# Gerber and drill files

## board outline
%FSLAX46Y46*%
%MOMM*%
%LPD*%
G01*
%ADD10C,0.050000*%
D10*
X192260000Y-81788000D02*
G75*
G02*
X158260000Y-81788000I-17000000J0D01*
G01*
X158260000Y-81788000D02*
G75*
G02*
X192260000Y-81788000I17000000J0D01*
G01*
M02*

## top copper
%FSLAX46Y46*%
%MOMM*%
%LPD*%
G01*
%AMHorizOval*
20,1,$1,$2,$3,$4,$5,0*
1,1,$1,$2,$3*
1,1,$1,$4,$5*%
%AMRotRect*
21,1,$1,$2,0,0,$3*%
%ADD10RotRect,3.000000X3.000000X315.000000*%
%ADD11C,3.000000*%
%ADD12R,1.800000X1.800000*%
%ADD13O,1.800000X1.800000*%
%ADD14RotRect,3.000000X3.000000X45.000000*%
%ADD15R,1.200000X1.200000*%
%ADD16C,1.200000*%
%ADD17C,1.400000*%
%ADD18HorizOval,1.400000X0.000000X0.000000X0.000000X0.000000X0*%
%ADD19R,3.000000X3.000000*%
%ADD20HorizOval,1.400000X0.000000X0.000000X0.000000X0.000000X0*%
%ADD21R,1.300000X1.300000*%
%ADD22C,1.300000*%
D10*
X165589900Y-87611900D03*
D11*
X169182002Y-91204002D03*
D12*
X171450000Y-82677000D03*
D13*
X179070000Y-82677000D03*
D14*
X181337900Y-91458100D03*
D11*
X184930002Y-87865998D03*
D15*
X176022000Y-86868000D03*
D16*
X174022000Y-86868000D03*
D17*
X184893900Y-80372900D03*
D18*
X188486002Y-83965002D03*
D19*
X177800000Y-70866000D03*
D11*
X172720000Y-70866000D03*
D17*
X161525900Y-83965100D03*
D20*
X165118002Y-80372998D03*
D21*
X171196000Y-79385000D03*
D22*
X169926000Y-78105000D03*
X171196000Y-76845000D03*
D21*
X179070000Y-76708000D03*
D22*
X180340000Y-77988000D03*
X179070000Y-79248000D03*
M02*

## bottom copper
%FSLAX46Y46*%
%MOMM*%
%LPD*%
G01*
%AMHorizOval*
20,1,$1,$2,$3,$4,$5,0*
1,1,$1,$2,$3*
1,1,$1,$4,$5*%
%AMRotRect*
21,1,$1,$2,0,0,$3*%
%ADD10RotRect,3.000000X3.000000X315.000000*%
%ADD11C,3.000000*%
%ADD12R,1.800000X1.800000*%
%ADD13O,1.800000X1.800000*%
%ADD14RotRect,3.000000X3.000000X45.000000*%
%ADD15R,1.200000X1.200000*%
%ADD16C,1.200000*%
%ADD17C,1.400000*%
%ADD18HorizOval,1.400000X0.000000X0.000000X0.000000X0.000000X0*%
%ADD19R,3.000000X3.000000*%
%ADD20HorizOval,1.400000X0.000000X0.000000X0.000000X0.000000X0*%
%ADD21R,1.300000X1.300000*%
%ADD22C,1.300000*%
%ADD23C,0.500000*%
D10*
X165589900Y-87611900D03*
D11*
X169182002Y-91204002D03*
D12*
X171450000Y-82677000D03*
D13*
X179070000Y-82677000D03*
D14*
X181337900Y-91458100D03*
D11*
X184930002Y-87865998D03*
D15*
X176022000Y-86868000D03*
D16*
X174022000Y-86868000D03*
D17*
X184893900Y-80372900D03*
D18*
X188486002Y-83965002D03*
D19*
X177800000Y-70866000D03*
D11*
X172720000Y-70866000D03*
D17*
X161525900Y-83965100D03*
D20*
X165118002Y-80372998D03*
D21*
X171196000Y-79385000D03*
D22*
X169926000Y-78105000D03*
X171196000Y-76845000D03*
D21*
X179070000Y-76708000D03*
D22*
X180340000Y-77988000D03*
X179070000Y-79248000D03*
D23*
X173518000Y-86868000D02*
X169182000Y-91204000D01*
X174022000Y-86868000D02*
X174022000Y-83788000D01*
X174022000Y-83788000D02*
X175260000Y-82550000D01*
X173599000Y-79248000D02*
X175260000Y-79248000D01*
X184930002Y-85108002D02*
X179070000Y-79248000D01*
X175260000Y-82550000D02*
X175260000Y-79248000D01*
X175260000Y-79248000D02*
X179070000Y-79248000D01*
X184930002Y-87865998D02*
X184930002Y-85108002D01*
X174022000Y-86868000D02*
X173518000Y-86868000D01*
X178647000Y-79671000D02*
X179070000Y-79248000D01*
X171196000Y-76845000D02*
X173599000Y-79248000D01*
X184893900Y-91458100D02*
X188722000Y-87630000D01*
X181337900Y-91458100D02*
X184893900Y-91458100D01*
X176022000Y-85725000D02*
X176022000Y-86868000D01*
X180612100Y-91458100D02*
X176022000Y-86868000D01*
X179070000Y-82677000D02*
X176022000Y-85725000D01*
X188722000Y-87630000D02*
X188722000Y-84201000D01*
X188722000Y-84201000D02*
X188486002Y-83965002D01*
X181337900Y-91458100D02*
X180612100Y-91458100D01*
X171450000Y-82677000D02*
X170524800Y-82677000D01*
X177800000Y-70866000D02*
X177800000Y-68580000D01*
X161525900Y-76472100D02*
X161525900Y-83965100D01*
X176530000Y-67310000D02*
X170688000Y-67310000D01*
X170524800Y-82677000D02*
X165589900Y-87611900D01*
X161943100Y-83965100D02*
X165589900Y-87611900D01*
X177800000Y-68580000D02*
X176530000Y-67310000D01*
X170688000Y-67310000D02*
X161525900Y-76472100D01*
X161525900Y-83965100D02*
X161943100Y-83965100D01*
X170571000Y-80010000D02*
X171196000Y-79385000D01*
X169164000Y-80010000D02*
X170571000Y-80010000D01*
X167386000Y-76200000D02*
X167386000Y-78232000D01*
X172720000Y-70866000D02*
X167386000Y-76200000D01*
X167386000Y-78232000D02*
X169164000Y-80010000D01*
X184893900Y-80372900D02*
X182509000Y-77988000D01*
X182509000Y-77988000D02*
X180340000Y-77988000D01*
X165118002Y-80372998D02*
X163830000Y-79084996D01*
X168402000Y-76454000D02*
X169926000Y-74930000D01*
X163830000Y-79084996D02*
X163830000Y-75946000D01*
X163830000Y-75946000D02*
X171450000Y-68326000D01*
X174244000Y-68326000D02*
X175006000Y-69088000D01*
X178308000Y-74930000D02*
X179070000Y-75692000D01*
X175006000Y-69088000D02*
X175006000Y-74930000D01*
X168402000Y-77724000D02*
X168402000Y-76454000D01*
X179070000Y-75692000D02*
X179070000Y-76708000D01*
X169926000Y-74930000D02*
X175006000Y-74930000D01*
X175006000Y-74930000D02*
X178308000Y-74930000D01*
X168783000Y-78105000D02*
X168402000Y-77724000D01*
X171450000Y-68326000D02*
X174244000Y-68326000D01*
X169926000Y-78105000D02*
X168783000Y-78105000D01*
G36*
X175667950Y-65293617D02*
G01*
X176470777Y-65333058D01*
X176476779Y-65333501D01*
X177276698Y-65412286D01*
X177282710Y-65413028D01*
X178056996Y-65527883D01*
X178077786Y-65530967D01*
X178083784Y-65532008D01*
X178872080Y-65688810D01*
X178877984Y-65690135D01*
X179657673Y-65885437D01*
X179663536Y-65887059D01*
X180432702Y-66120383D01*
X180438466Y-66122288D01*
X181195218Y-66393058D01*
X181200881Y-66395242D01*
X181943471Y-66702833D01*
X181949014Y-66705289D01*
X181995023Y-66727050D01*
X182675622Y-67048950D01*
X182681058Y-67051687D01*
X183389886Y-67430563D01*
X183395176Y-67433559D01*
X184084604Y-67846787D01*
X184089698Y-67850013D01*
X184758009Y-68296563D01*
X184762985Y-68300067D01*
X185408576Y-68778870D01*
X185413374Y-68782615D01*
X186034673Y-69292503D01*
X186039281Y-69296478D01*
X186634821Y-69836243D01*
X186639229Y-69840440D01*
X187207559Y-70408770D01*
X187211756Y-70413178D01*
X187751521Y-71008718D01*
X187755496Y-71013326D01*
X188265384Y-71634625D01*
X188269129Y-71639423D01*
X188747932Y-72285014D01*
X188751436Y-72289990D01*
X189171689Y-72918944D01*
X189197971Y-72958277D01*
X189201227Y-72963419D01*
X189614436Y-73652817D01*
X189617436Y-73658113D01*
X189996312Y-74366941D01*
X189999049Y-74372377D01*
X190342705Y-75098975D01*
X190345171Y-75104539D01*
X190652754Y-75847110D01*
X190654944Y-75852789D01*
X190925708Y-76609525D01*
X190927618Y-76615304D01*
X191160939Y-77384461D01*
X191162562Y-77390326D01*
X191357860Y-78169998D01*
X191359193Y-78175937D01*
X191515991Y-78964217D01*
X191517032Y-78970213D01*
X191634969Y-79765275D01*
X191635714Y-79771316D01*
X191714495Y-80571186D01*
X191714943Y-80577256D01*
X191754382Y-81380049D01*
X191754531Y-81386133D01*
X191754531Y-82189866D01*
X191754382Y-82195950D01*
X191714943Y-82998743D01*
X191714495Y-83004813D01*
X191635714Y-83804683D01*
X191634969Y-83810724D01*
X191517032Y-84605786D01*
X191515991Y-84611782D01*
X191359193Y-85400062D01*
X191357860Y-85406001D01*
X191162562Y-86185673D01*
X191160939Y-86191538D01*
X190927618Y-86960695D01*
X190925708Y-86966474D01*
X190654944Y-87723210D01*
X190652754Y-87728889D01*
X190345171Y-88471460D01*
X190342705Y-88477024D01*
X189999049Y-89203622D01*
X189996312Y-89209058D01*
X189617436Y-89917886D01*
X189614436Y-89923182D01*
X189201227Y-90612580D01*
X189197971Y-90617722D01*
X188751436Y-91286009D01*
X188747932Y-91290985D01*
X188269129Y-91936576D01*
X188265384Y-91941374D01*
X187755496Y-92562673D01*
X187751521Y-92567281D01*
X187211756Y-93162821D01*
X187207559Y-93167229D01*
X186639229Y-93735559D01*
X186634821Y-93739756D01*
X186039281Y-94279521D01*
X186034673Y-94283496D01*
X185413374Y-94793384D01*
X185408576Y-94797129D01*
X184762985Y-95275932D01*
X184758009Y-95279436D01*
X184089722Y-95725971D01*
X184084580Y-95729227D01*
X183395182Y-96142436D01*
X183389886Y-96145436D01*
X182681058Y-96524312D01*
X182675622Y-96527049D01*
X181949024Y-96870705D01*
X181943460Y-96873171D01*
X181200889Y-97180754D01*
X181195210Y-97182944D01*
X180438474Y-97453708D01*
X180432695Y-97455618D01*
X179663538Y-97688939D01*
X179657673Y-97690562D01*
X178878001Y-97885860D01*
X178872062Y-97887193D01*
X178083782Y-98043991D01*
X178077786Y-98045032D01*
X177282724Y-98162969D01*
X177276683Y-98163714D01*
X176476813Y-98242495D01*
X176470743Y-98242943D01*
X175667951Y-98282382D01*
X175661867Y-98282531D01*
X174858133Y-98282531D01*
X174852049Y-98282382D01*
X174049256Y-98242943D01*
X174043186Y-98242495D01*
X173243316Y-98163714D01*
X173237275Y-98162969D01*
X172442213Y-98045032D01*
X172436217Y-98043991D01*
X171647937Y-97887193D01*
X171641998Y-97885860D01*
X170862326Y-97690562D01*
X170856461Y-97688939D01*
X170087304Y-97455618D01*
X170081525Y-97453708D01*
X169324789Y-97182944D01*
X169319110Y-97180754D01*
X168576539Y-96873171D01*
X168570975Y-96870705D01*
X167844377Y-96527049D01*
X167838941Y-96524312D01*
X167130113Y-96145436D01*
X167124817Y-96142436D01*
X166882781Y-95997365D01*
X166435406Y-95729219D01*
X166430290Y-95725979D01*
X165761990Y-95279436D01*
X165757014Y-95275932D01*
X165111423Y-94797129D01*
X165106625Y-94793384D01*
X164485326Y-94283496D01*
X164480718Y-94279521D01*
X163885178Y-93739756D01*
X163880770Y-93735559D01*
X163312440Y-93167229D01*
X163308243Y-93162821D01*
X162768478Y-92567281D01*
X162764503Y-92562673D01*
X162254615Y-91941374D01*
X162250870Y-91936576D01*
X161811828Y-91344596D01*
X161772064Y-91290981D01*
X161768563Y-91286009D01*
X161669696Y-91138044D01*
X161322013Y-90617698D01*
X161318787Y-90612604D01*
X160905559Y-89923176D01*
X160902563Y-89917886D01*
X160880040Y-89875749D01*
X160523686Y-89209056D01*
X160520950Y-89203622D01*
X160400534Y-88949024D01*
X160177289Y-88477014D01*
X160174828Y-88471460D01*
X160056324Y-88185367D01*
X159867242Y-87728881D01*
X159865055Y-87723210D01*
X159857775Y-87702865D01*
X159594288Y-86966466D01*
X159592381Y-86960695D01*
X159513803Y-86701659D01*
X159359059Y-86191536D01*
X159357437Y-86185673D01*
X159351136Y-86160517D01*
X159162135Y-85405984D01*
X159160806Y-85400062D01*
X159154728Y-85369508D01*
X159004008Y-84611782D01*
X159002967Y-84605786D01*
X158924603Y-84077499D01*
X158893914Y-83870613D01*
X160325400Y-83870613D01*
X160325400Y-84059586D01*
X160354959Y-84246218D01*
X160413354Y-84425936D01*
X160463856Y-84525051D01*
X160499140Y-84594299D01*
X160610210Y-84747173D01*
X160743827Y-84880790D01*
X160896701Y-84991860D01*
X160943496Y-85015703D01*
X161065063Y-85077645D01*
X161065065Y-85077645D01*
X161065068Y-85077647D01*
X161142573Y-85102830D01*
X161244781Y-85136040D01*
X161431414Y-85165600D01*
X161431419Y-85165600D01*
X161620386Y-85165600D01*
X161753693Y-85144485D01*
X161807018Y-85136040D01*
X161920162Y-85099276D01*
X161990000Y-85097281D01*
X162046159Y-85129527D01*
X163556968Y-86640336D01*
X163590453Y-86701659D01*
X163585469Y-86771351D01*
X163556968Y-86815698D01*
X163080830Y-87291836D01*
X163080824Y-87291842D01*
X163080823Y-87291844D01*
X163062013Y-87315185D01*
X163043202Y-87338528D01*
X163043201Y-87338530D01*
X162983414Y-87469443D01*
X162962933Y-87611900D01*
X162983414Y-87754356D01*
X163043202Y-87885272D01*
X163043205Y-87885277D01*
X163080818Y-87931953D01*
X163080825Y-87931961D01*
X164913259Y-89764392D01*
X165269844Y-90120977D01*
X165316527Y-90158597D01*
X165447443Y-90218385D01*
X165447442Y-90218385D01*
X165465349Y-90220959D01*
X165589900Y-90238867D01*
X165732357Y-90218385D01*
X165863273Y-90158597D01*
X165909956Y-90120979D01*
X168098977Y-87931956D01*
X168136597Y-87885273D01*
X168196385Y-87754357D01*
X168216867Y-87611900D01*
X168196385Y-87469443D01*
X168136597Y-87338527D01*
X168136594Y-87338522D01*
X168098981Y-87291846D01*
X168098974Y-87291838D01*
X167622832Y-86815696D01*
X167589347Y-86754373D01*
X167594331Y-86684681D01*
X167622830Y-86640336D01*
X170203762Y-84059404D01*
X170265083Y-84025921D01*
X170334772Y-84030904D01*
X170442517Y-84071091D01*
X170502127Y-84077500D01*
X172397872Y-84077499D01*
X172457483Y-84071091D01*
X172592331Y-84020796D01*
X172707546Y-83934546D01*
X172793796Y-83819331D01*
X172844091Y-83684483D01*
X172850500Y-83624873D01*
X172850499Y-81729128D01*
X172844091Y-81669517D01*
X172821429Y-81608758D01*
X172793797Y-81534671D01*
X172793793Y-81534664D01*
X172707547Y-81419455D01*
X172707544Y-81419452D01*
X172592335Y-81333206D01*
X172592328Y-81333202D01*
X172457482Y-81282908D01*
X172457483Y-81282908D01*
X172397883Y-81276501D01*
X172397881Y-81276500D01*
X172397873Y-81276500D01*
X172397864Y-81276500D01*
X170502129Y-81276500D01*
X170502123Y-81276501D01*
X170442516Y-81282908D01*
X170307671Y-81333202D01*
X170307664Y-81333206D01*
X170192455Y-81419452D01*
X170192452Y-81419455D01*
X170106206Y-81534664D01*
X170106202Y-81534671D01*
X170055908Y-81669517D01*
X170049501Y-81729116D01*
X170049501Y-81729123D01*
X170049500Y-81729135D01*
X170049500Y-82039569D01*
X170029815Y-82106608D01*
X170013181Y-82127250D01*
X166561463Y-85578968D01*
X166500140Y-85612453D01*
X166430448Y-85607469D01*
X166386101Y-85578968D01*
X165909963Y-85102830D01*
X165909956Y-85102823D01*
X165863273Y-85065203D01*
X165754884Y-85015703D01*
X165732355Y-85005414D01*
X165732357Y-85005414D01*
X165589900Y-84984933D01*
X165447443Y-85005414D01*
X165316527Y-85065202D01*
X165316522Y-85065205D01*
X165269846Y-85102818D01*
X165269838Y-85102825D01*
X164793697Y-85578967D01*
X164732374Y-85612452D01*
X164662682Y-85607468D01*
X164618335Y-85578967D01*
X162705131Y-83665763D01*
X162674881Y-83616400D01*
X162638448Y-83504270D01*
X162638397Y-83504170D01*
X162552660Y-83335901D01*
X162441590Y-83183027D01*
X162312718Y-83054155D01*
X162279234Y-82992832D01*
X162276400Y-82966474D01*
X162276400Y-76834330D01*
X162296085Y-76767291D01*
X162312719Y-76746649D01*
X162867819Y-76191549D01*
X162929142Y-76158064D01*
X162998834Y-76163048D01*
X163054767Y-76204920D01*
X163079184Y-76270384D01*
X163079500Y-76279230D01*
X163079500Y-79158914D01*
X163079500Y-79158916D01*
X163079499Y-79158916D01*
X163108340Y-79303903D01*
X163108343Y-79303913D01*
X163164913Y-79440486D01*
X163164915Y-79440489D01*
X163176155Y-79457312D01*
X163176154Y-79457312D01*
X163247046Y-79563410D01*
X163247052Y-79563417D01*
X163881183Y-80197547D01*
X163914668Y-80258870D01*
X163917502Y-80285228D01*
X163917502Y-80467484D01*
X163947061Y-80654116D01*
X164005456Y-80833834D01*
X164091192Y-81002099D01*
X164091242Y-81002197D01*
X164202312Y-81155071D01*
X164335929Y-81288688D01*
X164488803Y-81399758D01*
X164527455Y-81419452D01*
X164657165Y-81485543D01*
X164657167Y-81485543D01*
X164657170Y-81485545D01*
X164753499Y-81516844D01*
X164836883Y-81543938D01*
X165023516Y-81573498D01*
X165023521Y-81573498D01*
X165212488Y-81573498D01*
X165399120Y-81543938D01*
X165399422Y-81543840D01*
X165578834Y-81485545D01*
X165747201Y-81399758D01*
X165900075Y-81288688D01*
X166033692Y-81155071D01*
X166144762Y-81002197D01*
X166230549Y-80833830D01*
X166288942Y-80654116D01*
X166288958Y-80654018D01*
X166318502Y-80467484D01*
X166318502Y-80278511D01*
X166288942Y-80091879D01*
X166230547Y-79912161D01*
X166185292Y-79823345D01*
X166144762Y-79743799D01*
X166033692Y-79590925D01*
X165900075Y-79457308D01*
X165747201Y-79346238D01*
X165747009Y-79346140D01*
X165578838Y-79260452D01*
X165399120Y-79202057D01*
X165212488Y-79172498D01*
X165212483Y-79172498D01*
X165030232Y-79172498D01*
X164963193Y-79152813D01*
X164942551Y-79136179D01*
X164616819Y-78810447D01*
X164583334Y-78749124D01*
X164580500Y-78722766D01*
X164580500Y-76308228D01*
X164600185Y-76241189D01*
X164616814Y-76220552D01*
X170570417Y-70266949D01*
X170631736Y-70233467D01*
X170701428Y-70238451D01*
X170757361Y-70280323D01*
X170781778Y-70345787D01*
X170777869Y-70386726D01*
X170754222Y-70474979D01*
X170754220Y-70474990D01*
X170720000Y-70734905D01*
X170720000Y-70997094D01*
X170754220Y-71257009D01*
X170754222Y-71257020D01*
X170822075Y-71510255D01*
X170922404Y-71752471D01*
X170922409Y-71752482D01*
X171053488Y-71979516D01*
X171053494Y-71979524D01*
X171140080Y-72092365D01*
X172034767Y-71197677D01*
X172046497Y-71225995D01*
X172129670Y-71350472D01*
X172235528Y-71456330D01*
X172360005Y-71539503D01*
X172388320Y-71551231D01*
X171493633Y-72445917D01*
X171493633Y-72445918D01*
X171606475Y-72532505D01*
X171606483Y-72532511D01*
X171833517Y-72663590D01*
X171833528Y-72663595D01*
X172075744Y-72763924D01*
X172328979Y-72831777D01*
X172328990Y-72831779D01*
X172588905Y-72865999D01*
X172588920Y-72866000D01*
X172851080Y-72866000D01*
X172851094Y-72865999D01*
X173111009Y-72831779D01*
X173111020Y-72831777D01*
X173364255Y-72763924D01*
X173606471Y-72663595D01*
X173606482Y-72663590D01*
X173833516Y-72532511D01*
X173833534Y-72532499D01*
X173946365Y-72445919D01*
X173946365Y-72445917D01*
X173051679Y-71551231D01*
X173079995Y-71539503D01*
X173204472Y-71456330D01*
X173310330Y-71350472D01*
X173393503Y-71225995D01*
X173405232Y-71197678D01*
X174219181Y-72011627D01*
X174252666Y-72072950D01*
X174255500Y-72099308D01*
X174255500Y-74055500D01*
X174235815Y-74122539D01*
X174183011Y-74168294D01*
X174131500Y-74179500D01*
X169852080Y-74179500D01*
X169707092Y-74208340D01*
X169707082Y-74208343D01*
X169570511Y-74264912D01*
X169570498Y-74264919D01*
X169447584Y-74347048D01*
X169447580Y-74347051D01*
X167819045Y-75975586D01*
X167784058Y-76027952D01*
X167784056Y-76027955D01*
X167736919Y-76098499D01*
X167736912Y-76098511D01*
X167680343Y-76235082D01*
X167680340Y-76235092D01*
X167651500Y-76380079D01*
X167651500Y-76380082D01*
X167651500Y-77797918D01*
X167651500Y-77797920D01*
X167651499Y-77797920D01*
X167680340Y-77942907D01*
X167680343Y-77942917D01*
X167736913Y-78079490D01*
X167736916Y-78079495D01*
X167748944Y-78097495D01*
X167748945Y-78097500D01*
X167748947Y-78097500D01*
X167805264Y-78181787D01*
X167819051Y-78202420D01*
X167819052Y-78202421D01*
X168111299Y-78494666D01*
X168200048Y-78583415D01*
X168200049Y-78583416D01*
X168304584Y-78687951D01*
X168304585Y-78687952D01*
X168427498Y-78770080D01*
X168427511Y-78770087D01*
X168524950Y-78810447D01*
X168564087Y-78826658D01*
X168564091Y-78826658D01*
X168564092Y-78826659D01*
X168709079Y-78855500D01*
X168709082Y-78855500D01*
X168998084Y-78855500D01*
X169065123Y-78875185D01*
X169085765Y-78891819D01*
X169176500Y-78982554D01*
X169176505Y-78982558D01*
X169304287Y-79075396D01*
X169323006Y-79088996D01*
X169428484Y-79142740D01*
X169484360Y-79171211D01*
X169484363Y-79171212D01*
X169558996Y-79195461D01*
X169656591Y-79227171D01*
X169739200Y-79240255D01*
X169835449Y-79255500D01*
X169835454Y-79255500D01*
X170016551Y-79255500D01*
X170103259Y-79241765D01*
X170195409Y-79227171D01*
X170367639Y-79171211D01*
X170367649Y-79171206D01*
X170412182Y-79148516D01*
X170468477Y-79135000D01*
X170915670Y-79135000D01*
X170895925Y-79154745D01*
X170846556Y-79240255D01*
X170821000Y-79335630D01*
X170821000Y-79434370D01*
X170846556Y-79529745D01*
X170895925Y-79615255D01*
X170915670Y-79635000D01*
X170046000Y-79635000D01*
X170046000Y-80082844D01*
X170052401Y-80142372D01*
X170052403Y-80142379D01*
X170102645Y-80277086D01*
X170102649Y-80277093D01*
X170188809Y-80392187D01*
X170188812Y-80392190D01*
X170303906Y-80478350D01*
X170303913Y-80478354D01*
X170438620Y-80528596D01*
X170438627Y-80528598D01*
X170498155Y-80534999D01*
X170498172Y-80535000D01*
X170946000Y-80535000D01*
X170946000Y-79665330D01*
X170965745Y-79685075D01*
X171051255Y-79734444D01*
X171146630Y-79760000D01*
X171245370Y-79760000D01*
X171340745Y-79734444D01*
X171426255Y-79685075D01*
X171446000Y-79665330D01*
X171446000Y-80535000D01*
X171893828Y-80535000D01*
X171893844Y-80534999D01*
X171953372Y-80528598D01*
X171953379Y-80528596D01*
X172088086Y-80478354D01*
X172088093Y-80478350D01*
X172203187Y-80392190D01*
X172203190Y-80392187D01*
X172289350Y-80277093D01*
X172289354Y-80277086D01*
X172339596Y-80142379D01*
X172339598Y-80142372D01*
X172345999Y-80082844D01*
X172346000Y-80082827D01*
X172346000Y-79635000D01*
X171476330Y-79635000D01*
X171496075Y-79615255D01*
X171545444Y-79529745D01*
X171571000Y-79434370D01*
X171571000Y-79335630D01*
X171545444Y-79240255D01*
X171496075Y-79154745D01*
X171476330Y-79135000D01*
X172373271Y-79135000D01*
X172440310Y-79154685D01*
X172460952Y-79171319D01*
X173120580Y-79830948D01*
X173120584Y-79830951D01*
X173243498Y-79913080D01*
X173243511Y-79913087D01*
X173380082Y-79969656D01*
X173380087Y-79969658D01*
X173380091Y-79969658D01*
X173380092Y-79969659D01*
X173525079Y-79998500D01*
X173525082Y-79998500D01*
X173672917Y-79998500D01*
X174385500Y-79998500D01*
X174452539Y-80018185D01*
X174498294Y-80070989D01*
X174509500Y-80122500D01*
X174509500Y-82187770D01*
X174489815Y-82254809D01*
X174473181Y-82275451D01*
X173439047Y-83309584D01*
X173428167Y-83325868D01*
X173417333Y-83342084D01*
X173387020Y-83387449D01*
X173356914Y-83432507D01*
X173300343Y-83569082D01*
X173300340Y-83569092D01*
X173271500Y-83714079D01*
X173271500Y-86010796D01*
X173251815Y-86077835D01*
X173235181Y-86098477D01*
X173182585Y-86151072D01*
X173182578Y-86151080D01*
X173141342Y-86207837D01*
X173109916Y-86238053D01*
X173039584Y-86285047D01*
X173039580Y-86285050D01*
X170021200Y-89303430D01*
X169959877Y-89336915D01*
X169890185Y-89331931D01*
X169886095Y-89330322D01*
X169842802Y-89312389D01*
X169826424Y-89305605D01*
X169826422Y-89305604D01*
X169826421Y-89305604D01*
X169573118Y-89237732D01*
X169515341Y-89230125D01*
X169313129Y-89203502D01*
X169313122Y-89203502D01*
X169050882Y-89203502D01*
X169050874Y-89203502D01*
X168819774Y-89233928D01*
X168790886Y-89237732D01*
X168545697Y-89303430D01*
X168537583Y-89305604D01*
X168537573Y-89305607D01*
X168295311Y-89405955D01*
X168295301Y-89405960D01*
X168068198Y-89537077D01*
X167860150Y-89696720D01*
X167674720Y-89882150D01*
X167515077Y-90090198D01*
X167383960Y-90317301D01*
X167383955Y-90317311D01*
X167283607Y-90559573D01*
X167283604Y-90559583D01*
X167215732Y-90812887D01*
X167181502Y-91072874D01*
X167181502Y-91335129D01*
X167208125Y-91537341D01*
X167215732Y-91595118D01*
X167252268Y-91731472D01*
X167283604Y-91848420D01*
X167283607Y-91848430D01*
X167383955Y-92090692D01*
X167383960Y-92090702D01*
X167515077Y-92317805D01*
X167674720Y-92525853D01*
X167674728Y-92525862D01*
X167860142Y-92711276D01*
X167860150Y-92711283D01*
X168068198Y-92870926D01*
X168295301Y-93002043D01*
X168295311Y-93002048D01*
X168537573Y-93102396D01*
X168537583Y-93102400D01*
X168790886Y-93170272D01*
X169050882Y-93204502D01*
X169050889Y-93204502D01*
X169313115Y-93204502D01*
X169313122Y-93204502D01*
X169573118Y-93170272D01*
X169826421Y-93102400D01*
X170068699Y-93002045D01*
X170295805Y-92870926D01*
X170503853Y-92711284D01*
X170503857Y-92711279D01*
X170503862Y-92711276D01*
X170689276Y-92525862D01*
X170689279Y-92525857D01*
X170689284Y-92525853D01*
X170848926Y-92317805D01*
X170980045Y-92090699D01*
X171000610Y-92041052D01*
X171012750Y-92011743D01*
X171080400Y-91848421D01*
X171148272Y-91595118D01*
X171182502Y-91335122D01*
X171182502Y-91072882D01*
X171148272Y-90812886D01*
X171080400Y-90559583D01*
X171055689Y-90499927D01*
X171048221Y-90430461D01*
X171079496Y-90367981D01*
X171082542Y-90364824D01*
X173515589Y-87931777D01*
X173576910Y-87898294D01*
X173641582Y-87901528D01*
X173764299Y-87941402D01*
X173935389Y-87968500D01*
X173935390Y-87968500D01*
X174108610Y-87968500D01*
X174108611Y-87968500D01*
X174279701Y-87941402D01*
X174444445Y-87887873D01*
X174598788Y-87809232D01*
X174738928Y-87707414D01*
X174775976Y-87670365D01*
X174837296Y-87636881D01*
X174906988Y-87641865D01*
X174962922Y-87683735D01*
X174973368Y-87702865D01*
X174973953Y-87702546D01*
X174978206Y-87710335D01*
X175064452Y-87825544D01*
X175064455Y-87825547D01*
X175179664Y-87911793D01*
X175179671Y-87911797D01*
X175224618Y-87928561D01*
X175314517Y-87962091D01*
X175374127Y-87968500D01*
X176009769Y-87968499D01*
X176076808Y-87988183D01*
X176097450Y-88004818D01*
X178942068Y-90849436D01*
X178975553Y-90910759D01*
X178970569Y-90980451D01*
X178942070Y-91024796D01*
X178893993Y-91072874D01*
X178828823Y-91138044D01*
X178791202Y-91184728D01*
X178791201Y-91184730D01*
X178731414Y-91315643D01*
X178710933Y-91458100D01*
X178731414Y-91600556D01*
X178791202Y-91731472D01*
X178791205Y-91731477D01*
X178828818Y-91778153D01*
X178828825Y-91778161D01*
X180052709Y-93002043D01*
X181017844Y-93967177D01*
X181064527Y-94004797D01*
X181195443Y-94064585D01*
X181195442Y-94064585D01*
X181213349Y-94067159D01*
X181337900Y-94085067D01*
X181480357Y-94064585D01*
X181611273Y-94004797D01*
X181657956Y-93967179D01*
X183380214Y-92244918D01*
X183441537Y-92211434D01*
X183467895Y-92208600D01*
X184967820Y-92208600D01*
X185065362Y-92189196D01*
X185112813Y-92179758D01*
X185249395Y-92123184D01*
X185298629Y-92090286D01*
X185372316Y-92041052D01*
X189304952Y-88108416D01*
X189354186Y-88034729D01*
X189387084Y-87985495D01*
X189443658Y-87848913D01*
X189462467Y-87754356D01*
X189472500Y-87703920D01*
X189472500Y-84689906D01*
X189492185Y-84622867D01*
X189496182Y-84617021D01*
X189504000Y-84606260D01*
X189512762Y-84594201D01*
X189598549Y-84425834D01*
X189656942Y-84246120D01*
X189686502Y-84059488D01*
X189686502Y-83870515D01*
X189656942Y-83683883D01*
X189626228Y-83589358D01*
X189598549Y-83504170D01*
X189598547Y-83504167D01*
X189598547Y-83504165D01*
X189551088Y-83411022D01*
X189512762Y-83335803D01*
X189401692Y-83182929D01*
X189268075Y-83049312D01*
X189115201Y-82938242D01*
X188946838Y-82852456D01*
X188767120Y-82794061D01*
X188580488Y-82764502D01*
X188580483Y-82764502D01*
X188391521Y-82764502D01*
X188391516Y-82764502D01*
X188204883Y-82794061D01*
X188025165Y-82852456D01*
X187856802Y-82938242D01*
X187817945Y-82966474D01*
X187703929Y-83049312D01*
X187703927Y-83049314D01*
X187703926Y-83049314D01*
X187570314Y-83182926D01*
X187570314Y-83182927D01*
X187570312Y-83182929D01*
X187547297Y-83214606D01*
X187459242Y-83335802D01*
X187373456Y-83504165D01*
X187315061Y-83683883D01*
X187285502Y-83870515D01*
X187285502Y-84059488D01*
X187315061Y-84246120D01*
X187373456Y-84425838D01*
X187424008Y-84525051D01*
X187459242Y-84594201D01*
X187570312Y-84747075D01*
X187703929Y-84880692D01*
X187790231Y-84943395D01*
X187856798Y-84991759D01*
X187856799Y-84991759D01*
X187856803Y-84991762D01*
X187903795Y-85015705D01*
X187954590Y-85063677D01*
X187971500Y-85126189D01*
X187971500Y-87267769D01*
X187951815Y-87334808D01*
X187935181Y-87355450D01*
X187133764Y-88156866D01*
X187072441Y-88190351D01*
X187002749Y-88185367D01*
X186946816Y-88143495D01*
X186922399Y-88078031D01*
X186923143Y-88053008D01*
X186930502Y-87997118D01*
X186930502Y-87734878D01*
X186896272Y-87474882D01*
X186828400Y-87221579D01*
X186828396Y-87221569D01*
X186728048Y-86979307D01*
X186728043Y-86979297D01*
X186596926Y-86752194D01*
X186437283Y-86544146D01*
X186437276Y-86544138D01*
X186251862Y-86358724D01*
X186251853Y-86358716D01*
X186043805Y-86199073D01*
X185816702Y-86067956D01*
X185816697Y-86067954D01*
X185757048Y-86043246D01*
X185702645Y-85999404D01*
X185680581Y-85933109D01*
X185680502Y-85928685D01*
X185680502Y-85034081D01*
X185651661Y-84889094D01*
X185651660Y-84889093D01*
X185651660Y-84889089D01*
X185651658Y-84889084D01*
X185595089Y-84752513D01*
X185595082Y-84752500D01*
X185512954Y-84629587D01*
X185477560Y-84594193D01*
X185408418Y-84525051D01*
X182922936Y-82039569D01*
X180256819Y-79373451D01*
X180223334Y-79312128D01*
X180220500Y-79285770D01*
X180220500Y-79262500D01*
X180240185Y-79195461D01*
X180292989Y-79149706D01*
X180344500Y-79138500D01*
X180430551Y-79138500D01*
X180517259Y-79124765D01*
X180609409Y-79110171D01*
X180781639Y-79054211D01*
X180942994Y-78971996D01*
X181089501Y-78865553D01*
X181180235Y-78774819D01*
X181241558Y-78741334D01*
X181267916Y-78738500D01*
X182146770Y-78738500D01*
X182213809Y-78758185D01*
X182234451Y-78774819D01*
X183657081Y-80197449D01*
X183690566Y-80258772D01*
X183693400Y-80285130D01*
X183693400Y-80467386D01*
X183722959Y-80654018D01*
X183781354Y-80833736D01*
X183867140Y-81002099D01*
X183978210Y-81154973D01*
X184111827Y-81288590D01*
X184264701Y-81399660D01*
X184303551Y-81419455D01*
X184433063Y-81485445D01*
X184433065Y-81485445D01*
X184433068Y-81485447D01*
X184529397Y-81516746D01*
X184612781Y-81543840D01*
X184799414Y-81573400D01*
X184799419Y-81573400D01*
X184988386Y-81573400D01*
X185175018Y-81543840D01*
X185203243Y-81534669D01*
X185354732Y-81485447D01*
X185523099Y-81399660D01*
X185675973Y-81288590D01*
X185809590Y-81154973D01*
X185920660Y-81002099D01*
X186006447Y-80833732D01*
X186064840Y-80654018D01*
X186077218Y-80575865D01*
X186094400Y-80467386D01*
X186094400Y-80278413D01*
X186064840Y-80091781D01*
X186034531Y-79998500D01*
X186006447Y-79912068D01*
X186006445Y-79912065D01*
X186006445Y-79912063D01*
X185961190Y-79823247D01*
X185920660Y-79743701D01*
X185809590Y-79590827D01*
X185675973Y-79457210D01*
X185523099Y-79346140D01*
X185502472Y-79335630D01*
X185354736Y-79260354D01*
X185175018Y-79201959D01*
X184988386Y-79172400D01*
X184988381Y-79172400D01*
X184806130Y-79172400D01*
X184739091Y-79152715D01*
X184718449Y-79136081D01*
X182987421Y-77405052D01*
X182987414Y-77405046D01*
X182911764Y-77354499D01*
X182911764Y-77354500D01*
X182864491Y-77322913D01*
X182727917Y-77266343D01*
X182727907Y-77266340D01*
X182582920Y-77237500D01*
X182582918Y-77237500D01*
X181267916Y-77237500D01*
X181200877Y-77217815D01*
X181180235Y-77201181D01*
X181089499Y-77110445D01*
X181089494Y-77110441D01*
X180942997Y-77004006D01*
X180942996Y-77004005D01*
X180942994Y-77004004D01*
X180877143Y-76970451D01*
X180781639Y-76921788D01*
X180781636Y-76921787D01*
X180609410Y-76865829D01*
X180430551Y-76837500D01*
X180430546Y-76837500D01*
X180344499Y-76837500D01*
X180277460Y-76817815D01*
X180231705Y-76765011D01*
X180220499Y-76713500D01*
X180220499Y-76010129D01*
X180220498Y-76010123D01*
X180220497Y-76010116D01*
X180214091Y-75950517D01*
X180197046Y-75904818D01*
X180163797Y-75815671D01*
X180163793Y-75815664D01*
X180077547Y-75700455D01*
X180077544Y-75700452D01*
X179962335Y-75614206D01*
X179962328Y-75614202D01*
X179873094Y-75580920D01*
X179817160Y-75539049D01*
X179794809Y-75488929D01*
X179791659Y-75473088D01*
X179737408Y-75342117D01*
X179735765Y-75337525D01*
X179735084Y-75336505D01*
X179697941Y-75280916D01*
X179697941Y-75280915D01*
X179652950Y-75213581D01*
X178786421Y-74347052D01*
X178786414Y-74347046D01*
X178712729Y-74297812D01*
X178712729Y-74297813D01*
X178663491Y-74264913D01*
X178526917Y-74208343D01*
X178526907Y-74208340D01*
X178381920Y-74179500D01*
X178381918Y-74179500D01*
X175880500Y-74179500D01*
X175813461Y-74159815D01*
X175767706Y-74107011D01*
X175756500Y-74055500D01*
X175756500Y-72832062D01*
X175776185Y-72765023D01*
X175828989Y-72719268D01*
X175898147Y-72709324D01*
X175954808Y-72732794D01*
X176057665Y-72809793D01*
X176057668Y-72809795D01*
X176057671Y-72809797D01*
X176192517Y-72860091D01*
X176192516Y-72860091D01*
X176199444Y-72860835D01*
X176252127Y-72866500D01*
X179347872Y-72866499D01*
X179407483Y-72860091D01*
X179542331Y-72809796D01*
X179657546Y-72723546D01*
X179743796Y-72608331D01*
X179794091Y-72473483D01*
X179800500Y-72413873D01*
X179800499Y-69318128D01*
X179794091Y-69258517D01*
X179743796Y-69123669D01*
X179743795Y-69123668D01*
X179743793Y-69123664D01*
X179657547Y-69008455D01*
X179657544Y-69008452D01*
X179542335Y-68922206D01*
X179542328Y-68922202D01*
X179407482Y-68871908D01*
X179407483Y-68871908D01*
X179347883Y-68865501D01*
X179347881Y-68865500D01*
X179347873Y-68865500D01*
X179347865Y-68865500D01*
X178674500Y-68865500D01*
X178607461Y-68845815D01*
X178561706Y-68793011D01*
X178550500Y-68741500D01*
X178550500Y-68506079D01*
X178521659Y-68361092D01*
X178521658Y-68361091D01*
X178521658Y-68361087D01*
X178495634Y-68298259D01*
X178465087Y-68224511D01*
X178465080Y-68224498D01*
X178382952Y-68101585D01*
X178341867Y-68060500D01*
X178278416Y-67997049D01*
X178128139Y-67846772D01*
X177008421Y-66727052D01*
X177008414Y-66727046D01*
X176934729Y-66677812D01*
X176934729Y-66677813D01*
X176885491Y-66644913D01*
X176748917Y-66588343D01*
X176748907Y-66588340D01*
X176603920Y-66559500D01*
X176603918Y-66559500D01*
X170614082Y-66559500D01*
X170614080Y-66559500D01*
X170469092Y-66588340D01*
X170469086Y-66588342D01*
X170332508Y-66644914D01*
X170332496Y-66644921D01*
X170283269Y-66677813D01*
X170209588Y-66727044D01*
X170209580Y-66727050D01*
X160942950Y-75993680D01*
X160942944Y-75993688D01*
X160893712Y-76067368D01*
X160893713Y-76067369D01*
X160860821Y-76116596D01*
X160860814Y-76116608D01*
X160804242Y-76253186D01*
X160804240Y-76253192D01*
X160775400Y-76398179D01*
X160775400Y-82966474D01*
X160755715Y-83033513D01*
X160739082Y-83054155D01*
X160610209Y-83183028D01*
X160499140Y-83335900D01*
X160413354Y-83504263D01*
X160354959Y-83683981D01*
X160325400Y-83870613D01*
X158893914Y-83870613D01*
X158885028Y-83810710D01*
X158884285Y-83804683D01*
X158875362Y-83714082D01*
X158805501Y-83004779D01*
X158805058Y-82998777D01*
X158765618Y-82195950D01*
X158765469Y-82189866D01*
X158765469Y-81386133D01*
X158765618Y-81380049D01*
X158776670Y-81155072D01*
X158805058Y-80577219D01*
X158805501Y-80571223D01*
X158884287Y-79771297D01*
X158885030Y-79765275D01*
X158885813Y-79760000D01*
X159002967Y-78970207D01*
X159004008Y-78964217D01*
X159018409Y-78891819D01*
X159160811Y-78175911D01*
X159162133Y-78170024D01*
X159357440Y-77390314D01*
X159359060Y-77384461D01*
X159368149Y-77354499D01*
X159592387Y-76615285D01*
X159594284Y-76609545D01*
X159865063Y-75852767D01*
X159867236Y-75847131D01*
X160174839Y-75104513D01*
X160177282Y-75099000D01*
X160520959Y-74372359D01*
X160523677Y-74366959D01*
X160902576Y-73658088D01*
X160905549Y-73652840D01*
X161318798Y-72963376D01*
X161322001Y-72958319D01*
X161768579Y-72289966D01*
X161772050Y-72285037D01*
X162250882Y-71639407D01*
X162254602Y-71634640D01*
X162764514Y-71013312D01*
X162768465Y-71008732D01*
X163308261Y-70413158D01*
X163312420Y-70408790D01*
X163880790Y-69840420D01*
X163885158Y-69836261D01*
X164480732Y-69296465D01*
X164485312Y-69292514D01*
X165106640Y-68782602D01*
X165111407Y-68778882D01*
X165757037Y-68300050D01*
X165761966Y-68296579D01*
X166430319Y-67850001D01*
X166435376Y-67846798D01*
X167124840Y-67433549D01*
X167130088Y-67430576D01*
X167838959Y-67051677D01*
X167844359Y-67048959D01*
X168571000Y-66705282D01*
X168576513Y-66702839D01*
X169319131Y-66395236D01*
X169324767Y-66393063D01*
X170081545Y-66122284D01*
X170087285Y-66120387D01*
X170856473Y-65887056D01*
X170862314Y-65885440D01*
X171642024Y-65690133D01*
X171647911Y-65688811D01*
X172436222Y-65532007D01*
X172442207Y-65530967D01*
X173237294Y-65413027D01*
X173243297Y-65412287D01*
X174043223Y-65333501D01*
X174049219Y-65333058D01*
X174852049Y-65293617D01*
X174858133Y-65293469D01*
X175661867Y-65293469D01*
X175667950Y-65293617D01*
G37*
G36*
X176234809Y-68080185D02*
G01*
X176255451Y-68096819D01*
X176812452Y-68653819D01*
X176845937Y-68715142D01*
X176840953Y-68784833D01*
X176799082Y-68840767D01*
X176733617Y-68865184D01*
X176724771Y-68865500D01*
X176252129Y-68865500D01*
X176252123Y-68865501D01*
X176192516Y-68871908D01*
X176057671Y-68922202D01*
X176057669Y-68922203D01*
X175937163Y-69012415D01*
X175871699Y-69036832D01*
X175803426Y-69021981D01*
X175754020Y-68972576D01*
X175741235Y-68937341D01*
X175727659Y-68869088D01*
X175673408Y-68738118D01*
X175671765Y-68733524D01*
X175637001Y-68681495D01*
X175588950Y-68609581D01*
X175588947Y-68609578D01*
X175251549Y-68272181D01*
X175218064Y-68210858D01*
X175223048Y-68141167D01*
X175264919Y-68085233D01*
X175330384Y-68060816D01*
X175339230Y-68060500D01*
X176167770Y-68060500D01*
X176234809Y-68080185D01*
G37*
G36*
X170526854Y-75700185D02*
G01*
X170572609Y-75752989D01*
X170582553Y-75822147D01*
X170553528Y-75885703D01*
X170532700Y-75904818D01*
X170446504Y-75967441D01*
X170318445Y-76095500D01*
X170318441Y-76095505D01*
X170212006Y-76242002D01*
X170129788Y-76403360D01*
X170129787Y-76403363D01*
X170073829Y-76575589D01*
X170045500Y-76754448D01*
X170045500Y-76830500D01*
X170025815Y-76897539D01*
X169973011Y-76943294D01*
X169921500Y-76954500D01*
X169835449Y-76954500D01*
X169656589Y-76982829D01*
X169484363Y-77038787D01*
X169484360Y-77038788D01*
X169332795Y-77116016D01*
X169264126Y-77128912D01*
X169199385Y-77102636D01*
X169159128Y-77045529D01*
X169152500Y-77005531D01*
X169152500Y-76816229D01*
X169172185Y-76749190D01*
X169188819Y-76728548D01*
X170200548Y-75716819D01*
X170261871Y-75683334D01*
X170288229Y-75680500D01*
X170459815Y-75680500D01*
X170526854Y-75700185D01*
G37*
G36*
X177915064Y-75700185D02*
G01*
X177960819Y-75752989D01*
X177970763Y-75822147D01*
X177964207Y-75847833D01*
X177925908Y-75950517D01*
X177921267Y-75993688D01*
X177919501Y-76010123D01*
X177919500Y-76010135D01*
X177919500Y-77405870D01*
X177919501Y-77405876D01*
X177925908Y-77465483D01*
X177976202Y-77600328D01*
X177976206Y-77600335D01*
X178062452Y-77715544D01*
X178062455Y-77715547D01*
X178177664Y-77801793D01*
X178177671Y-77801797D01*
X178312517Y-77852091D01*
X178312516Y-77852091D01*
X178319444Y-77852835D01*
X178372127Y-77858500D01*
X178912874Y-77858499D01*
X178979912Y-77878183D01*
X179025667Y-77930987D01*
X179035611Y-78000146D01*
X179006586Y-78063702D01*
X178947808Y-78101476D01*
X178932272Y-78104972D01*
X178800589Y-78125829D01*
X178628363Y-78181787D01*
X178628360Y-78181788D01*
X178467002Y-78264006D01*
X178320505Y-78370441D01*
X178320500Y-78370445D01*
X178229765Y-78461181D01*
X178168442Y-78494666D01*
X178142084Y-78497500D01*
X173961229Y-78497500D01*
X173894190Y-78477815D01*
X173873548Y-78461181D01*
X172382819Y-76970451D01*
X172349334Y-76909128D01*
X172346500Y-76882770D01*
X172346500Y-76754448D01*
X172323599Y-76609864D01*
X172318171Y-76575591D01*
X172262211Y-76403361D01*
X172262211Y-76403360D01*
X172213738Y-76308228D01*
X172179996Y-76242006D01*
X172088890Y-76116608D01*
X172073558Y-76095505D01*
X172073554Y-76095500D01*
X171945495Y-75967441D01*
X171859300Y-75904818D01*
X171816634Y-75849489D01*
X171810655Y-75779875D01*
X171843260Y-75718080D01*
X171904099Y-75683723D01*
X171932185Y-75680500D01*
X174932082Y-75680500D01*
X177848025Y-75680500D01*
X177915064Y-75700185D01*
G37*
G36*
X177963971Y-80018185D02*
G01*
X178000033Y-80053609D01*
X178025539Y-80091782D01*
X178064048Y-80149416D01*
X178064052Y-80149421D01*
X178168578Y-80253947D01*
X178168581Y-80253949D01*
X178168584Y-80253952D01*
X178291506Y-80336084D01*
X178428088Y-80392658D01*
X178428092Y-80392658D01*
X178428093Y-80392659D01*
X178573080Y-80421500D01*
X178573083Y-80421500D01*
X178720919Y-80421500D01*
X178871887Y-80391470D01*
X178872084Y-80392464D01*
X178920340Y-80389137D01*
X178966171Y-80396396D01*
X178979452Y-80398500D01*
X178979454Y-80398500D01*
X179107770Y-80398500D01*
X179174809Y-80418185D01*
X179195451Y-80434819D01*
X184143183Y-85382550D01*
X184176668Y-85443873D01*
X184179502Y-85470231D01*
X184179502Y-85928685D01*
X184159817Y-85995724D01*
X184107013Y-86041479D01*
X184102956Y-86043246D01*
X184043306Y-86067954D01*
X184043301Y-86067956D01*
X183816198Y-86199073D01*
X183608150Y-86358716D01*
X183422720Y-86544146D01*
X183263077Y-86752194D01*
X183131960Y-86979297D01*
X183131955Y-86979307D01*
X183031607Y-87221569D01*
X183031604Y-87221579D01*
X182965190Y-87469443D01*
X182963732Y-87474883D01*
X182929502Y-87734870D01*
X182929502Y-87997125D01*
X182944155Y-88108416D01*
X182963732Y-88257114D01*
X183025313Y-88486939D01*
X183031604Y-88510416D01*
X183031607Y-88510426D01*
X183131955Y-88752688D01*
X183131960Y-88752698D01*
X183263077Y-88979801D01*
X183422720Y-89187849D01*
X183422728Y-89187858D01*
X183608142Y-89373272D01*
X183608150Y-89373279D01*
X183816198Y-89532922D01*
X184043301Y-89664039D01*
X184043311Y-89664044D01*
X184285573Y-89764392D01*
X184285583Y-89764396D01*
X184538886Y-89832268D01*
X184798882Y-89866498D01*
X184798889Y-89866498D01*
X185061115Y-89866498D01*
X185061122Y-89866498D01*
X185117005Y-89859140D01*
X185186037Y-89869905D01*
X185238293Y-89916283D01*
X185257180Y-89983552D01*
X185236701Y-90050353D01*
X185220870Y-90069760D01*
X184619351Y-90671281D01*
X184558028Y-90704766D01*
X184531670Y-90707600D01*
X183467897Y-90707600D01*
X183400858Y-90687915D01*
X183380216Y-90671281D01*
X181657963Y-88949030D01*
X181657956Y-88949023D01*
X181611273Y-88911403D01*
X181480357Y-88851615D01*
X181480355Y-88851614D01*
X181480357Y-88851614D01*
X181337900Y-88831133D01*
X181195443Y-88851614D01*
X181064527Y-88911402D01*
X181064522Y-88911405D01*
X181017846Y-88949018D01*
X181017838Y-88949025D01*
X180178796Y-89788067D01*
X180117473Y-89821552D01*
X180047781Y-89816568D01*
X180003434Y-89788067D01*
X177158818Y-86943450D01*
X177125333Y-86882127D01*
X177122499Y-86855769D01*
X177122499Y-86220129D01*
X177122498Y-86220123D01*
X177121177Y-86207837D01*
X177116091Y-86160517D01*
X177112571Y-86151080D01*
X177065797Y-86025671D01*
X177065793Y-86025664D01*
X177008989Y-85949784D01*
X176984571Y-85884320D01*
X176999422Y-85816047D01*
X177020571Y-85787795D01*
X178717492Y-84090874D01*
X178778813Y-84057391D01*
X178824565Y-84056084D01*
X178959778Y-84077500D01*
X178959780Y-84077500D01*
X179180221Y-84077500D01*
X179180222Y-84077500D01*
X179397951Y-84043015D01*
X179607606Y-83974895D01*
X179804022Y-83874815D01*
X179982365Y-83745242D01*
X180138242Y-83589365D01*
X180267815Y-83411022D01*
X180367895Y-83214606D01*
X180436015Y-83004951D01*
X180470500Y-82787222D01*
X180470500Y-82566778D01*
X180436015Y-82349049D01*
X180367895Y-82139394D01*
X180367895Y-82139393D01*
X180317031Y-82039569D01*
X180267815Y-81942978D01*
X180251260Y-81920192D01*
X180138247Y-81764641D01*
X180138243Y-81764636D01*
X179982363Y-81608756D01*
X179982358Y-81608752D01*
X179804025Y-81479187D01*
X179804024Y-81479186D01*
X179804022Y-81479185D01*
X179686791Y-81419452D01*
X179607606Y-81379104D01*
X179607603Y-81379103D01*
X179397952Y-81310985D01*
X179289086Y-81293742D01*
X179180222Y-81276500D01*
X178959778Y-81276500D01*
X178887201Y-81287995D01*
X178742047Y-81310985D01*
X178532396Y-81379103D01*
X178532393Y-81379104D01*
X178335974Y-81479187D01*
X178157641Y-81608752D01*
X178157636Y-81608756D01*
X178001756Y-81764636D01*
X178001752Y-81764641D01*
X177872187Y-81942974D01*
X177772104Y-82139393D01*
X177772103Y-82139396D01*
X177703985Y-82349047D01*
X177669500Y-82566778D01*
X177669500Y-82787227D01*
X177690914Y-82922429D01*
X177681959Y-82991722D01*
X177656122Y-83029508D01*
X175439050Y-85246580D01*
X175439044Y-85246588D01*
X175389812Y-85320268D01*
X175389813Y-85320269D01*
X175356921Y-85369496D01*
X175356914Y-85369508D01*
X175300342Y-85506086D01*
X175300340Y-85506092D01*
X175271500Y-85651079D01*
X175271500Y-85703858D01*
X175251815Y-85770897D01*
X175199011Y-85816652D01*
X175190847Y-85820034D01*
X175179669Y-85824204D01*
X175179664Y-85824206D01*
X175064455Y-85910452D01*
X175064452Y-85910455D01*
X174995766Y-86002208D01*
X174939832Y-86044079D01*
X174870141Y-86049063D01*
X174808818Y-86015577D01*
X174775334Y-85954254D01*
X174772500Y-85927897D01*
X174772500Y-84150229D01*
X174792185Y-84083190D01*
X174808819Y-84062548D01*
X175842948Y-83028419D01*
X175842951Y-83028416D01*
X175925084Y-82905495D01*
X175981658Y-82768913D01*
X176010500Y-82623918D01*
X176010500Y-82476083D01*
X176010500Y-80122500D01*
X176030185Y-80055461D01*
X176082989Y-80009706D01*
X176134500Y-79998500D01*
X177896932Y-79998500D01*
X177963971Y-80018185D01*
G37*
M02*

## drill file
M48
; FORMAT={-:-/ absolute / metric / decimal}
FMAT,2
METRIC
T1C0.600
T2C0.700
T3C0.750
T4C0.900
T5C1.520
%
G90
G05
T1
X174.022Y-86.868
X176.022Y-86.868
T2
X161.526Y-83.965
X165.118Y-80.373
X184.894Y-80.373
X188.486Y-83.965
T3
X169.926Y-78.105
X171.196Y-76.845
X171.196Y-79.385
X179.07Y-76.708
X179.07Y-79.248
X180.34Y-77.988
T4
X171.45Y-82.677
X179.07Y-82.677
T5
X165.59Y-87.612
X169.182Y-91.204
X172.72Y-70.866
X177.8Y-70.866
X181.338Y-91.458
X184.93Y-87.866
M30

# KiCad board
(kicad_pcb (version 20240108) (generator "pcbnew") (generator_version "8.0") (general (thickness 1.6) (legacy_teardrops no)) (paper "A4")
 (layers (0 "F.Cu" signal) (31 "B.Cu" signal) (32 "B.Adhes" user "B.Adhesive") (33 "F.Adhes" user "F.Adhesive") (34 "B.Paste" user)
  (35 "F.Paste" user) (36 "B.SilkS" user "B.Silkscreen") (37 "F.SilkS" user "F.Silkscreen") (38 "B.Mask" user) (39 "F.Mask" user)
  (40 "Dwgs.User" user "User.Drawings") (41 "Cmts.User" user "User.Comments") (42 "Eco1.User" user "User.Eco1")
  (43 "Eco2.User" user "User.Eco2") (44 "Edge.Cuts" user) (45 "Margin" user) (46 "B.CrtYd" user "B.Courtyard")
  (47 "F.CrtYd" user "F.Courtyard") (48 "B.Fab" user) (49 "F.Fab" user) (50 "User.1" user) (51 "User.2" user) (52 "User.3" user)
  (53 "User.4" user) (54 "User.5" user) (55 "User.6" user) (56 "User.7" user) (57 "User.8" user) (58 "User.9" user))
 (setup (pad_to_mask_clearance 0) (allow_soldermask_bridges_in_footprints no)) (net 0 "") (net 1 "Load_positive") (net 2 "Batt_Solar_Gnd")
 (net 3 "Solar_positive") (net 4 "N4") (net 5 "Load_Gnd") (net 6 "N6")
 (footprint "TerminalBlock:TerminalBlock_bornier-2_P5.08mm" (layer "F.Cu") (at 165.5899 87.6119 -45)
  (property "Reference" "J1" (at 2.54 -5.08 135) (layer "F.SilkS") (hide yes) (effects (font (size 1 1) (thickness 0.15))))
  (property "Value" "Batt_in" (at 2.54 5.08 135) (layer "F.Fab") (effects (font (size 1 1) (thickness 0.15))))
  (pad "1" thru_hole rect (at 0 0 315) (size 3 3) (drill 1.52) (layers "*.Cu" "*.Mask") (remove_unused_layers no) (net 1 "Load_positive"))
  (pad "2" thru_hole circle (at 5.079999 0 315) (size 3 3) (drill 1.52) (layers "*.Cu" "*.Mask") (remove_unused_layers no)
   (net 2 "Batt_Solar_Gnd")))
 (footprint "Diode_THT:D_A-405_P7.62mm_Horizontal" (layer "F.Cu") (at 171.45 82.677)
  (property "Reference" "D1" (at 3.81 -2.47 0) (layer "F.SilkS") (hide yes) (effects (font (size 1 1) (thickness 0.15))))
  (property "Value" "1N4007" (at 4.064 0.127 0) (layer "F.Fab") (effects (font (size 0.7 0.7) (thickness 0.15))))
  (pad "1" thru_hole rect (at 0 0) (size 1.8 1.8) (drill 0.9) (layers "*.Cu" "*.Mask") (remove_unused_layers no) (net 1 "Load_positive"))
  (pad "2" thru_hole oval (at 7.62 0) (size 1.8 1.8) (drill 0.9) (layers "*.Cu" "*.Mask") (remove_unused_layers no) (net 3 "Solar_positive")))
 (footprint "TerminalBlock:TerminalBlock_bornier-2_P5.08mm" (layer "F.Cu") (at 181.3379 91.4581 45)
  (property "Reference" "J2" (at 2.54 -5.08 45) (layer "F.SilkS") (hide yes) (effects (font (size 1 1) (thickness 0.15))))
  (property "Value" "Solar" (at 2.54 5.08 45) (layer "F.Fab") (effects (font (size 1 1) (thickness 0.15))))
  (pad "1" thru_hole rect (at 0 0 45) (size 3 3) (drill 1.52) (layers "*.Cu" "*.Mask") (remove_unused_layers no) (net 3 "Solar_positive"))
  (pad "2" thru_hole circle (at 5.079999 0 45) (size 3 3) (drill 1.52) (layers "*.Cu" "*.Mask") (remove_unused_layers no)
   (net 2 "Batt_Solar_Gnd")))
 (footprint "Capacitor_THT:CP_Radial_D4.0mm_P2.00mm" (layer "F.Cu") (at 176.022 86.868 180)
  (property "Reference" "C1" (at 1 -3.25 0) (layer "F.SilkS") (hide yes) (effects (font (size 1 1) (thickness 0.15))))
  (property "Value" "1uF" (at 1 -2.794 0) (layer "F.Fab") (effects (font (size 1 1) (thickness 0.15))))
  (pad "1" thru_hole rect (at 0 0 180) (size 1.2 1.2) (drill 0.6) (layers "*.Cu" "*.Mask") (remove_unused_layers no)
   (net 3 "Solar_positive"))
  (pad "2" thru_hole circle (at 2 0 180) (size 1.2 1.2) (drill 0.6) (layers "*.Cu" "*.Mask") (remove_unused_layers no)
   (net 2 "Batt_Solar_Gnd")))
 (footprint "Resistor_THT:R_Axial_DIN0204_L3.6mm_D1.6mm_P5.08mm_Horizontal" (layer "F.Cu") (at 184.8939 80.3729 -45)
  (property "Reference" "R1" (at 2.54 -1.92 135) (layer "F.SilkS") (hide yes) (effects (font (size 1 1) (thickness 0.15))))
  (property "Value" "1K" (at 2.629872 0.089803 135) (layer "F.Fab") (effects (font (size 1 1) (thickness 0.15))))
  (pad "1" thru_hole circle (at 0 0 315) (size 1.4 1.4) (drill 0.7) (layers "*.Cu" "*.Mask") (remove_unused_layers no) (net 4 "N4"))
  (pad "2" thru_hole oval (at 5.079999 0 315) (size 1.4 1.4) (drill 0.7) (layers "*.Cu" "*.Mask") (remove_unused_layers no)
   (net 3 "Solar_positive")))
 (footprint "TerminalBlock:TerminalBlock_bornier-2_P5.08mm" (layer "F.Cu") (at 177.8 70.866 180)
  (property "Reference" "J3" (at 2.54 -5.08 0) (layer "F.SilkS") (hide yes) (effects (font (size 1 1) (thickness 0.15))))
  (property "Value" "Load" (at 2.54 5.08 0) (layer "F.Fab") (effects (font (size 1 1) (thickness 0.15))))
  (pad "1" thru_hole rect (at 0 0 180) (size 3 3) (drill 1.52) (layers "*.Cu" "*.Mask") (remove_unused_layers no) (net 1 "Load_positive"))
  (pad "2" thru_hole circle (at 5.08 0 180) (size 3 3) (drill 1.52) (layers "*.Cu" "*.Mask") (remove_unused_layers no) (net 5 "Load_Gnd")))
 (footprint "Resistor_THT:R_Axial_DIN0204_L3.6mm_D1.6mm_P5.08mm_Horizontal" (layer "F.Cu") (at 161.5259 83.9651 45)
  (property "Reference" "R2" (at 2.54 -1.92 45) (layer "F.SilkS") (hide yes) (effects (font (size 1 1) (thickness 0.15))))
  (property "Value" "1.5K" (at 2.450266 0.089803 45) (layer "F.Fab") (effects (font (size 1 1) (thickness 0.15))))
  (pad "1" thru_hole circle (at 0 0 45) (size 1.4 1.4) (drill 0.7) (layers "*.Cu" "*.Mask") (remove_unused_layers no)
   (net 1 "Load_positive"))
  (pad "2" thru_hole oval (at 5.079999 0 45) (size 1.4 1.4) (drill 0.7) (layers "*.Cu" "*.Mask") (remove_unused_layers no) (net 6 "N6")))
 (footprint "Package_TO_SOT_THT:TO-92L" (layer "F.Cu") (at 171.196 79.385 90)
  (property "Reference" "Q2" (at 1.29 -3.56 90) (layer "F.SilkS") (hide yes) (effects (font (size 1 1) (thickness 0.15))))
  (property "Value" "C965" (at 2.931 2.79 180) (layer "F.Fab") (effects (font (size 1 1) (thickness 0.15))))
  (pad "1" thru_hole rect (at 0 0 90) (size 1.3 1.3) (drill 0.75) (layers "*.Cu" "*.Mask") (remove_unused_layers no) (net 5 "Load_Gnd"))
  (pad "2" thru_hole circle (at 1.28 -1.27 90) (size 1.3 1.3) (drill 0.75) (layers "*.Cu" "*.Mask") (remove_unused_layers no) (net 6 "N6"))
  (pad "3" thru_hole circle (at 2.54 0 90) (size 1.3 1.3) (drill 0.75) (layers "*.Cu" "*.Mask") (remove_unused_layers no)
   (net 2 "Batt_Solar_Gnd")))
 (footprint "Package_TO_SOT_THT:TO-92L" (layer "F.Cu") (at 179.07 76.708 -90)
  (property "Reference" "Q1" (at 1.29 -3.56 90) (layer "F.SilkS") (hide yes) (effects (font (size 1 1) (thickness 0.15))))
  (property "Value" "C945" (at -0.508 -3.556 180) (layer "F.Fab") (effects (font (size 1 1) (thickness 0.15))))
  (pad "1" thru_hole rect (at 0 0 270) (size 1.3 1.3) (drill 0.75) (layers "*.Cu" "*.Mask") (remove_unused_layers no) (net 6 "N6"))
  (pad "2" thru_hole circle (at 1.28 -1.27 270) (size 1.3 1.3) (drill 0.75) (layers "*.Cu" "*.Mask") (remove_unused_layers no) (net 4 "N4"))
  (pad "3" thru_hole circle (at 2.54 0 270) (size 1.3 1.3) (drill 0.75) (layers "*.Cu" "*.Mask") (remove_unused_layers no)
   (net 2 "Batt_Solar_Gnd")))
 (gr_circle (center 175.26 81.788) (end 192.26 81.788) (stroke (width 0.05) (type default)) (fill none) (layer "Edge.Cuts"))
 (segment (start 173.518 86.868) (end 169.182 91.204) (width 0.5) (layer "B.Cu") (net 2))
 (segment (start 174.022 86.868) (end 174.022 83.788) (width 0.5) (layer "B.Cu") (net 2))
 (segment (start 174.022 83.788) (end 175.26 82.55) (width 0.5) (layer "B.Cu") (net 2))
 (segment (start 173.599 79.248) (end 175.26 79.248) (width 0.5) (layer "B.Cu") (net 2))
 (segment (start 184.930002 85.108002) (end 179.07 79.248) (width 0.5) (layer "B.Cu") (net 2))
 (segment (start 175.26 82.55) (end 175.26 79.248) (width 0.5) (layer "B.Cu") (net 2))
 (segment (start 175.26 79.248) (end 179.07 79.248) (width 0.5) (layer "B.Cu") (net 2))
 (segment (start 184.930002 87.865998) (end 184.930002 85.108002) (width 0.5) (layer "B.Cu") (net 2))
 (segment (start 174.022 86.868) (end 173.518 86.868) (width 0.5) (layer "B.Cu") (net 2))
 (segment (start 178.647 79.671) (end 179.07 79.248) (width 0.5) (layer "B.Cu") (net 2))
 (segment (start 171.196 76.845) (end 173.599 79.248) (width 0.5) (layer "B.Cu") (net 2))
 (segment (start 184.8939 91.4581) (end 188.722 87.63) (width 0.5) (layer "B.Cu") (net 3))
 (segment (start 181.3379 91.4581) (end 184.8939 91.4581) (width 0.5) (layer "B.Cu") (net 3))
 (segment (start 176.022 85.725) (end 176.022 86.868) (width 0.5) (layer "B.Cu") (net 3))
 (segment (start 180.6121 91.4581) (end 176.022 86.868) (width 0.5) (layer "B.Cu") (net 3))
 (segment (start 179.07 82.677) (end 176.022 85.725) (width 0.5) (layer "B.Cu") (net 3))
 (segment (start 188.722 87.63) (end 188.722 84.201) (width 0.5) (layer "B.Cu") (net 3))
 (segment (start 188.722 84.201) (end 188.486002 83.965002) (width 0.5) (layer "B.Cu") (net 3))
 (segment (start 181.3379 91.4581) (end 180.6121 91.4581) (width 0.5) (layer "B.Cu") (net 3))
 (segment (start 171.45 82.677) (end 170.5248 82.677) (width 0.5) (layer "B.Cu") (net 1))
 (segment (start 177.8 70.866) (end 177.8 68.58) (width 0.5) (layer "B.Cu") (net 1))
 (segment (start 161.5259 76.4721) (end 161.5259 83.9651) (width 0.5) (layer "B.Cu") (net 1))
 (segment (start 176.53 67.31) (end 170.688 67.31) (width 0.5) (layer "B.Cu") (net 1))
 (segment (start 170.5248 82.677) (end 165.5899 87.6119) (width 0.5) (layer "B.Cu") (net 1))
 (segment (start 161.9431 83.9651) (end 165.5899 87.6119) (width 0.5) (layer "B.Cu") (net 1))
 (segment (start 177.8 68.58) (end 176.53 67.31) (width 0.5) (layer "B.Cu") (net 1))
 (segment (start 170.688 67.31) (end 161.5259 76.4721) (width 0.5) (layer "B.Cu") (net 1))
 (segment (start 161.5259 83.9651) (end 161.9431 83.9651) (width 0.5) (layer "B.Cu") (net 1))
 (segment (start 170.571 80.01) (end 171.196 79.385) (width 0.5) (layer "B.Cu") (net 5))
 (segment (start 169.164 80.01) (end 170.571 80.01) (width 0.5) (layer "B.Cu") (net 5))
 (segment (start 167.386 76.2) (end 167.386 78.232) (width 0.5) (layer "B.Cu") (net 5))
 (segment (start 172.72 70.866) (end 167.386 76.2) (width 0.5) (layer "B.Cu") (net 5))
 (segment (start 167.386 78.232) (end 169.164 80.01) (width 0.5) (layer "B.Cu") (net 5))
 (segment (start 184.8939 80.3729) (end 182.509 77.988) (width 0.5) (layer "B.Cu") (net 4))
 (segment (start 182.509 77.988) (end 180.34 77.988) (width 0.5) (layer "B.Cu") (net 4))
 (segment (start 165.118002 80.372998) (end 163.83 79.084996) (width 0.5) (layer "B.Cu") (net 6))
 (segment (start 168.402 76.454) (end 169.926 74.93) (width 0.5) (layer "B.Cu") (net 6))
 (segment (start 163.83 79.084996) (end 163.83 75.946) (width 0.5) (layer "B.Cu") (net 6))
 (segment (start 163.83 75.946) (end 171.45 68.326) (width 0.5) (layer "B.Cu") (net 6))
 (segment (start 174.244 68.326) (end 175.006 69.088) (width 0.5) (layer "B.Cu") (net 6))
 (segment (start 178.308 74.93) (end 179.07 75.692) (width 0.5) (layer "B.Cu") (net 6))
 (segment (start 175.006 69.088) (end 175.006 74.93) (width 0.5) (layer "B.Cu") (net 6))
 (segment (start 168.402 77.724) (end 168.402 76.454) (width 0.5) (layer "B.Cu") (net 6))
 (segment (start 179.07 75.692) (end 179.07 76.708) (width 0.5) (layer "B.Cu") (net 6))
 (segment (start 169.926 74.93) (end 175.006 74.93) (width 0.5) (layer "B.Cu") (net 6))
 (segment (start 175.006 74.93) (end 178.308 74.93) (width 0.5) (layer "B.Cu") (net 6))
 (segment (start 168.783 78.105) (end 168.402 77.724) (width 0.5) (layer "B.Cu") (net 6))
 (segment (start 171.45 68.326) (end 174.244 68.326) (width 0.5) (layer "B.Cu") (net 6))
 (segment (start 169.926 78.105) (end 168.783 78.105) (width 0.5) (layer "B.Cu") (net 6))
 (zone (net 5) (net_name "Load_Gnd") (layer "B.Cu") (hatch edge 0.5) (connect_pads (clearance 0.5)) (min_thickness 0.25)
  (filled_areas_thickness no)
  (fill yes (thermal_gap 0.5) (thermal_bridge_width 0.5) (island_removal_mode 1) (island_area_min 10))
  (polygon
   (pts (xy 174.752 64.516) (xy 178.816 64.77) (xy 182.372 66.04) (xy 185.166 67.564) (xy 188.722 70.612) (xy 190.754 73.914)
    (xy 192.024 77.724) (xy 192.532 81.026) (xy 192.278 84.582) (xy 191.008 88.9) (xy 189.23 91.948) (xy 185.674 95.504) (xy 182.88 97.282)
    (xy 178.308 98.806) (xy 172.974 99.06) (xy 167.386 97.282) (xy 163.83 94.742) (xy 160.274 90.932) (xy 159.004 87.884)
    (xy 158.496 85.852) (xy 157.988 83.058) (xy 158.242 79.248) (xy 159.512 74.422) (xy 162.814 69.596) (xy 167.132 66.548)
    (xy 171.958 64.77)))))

